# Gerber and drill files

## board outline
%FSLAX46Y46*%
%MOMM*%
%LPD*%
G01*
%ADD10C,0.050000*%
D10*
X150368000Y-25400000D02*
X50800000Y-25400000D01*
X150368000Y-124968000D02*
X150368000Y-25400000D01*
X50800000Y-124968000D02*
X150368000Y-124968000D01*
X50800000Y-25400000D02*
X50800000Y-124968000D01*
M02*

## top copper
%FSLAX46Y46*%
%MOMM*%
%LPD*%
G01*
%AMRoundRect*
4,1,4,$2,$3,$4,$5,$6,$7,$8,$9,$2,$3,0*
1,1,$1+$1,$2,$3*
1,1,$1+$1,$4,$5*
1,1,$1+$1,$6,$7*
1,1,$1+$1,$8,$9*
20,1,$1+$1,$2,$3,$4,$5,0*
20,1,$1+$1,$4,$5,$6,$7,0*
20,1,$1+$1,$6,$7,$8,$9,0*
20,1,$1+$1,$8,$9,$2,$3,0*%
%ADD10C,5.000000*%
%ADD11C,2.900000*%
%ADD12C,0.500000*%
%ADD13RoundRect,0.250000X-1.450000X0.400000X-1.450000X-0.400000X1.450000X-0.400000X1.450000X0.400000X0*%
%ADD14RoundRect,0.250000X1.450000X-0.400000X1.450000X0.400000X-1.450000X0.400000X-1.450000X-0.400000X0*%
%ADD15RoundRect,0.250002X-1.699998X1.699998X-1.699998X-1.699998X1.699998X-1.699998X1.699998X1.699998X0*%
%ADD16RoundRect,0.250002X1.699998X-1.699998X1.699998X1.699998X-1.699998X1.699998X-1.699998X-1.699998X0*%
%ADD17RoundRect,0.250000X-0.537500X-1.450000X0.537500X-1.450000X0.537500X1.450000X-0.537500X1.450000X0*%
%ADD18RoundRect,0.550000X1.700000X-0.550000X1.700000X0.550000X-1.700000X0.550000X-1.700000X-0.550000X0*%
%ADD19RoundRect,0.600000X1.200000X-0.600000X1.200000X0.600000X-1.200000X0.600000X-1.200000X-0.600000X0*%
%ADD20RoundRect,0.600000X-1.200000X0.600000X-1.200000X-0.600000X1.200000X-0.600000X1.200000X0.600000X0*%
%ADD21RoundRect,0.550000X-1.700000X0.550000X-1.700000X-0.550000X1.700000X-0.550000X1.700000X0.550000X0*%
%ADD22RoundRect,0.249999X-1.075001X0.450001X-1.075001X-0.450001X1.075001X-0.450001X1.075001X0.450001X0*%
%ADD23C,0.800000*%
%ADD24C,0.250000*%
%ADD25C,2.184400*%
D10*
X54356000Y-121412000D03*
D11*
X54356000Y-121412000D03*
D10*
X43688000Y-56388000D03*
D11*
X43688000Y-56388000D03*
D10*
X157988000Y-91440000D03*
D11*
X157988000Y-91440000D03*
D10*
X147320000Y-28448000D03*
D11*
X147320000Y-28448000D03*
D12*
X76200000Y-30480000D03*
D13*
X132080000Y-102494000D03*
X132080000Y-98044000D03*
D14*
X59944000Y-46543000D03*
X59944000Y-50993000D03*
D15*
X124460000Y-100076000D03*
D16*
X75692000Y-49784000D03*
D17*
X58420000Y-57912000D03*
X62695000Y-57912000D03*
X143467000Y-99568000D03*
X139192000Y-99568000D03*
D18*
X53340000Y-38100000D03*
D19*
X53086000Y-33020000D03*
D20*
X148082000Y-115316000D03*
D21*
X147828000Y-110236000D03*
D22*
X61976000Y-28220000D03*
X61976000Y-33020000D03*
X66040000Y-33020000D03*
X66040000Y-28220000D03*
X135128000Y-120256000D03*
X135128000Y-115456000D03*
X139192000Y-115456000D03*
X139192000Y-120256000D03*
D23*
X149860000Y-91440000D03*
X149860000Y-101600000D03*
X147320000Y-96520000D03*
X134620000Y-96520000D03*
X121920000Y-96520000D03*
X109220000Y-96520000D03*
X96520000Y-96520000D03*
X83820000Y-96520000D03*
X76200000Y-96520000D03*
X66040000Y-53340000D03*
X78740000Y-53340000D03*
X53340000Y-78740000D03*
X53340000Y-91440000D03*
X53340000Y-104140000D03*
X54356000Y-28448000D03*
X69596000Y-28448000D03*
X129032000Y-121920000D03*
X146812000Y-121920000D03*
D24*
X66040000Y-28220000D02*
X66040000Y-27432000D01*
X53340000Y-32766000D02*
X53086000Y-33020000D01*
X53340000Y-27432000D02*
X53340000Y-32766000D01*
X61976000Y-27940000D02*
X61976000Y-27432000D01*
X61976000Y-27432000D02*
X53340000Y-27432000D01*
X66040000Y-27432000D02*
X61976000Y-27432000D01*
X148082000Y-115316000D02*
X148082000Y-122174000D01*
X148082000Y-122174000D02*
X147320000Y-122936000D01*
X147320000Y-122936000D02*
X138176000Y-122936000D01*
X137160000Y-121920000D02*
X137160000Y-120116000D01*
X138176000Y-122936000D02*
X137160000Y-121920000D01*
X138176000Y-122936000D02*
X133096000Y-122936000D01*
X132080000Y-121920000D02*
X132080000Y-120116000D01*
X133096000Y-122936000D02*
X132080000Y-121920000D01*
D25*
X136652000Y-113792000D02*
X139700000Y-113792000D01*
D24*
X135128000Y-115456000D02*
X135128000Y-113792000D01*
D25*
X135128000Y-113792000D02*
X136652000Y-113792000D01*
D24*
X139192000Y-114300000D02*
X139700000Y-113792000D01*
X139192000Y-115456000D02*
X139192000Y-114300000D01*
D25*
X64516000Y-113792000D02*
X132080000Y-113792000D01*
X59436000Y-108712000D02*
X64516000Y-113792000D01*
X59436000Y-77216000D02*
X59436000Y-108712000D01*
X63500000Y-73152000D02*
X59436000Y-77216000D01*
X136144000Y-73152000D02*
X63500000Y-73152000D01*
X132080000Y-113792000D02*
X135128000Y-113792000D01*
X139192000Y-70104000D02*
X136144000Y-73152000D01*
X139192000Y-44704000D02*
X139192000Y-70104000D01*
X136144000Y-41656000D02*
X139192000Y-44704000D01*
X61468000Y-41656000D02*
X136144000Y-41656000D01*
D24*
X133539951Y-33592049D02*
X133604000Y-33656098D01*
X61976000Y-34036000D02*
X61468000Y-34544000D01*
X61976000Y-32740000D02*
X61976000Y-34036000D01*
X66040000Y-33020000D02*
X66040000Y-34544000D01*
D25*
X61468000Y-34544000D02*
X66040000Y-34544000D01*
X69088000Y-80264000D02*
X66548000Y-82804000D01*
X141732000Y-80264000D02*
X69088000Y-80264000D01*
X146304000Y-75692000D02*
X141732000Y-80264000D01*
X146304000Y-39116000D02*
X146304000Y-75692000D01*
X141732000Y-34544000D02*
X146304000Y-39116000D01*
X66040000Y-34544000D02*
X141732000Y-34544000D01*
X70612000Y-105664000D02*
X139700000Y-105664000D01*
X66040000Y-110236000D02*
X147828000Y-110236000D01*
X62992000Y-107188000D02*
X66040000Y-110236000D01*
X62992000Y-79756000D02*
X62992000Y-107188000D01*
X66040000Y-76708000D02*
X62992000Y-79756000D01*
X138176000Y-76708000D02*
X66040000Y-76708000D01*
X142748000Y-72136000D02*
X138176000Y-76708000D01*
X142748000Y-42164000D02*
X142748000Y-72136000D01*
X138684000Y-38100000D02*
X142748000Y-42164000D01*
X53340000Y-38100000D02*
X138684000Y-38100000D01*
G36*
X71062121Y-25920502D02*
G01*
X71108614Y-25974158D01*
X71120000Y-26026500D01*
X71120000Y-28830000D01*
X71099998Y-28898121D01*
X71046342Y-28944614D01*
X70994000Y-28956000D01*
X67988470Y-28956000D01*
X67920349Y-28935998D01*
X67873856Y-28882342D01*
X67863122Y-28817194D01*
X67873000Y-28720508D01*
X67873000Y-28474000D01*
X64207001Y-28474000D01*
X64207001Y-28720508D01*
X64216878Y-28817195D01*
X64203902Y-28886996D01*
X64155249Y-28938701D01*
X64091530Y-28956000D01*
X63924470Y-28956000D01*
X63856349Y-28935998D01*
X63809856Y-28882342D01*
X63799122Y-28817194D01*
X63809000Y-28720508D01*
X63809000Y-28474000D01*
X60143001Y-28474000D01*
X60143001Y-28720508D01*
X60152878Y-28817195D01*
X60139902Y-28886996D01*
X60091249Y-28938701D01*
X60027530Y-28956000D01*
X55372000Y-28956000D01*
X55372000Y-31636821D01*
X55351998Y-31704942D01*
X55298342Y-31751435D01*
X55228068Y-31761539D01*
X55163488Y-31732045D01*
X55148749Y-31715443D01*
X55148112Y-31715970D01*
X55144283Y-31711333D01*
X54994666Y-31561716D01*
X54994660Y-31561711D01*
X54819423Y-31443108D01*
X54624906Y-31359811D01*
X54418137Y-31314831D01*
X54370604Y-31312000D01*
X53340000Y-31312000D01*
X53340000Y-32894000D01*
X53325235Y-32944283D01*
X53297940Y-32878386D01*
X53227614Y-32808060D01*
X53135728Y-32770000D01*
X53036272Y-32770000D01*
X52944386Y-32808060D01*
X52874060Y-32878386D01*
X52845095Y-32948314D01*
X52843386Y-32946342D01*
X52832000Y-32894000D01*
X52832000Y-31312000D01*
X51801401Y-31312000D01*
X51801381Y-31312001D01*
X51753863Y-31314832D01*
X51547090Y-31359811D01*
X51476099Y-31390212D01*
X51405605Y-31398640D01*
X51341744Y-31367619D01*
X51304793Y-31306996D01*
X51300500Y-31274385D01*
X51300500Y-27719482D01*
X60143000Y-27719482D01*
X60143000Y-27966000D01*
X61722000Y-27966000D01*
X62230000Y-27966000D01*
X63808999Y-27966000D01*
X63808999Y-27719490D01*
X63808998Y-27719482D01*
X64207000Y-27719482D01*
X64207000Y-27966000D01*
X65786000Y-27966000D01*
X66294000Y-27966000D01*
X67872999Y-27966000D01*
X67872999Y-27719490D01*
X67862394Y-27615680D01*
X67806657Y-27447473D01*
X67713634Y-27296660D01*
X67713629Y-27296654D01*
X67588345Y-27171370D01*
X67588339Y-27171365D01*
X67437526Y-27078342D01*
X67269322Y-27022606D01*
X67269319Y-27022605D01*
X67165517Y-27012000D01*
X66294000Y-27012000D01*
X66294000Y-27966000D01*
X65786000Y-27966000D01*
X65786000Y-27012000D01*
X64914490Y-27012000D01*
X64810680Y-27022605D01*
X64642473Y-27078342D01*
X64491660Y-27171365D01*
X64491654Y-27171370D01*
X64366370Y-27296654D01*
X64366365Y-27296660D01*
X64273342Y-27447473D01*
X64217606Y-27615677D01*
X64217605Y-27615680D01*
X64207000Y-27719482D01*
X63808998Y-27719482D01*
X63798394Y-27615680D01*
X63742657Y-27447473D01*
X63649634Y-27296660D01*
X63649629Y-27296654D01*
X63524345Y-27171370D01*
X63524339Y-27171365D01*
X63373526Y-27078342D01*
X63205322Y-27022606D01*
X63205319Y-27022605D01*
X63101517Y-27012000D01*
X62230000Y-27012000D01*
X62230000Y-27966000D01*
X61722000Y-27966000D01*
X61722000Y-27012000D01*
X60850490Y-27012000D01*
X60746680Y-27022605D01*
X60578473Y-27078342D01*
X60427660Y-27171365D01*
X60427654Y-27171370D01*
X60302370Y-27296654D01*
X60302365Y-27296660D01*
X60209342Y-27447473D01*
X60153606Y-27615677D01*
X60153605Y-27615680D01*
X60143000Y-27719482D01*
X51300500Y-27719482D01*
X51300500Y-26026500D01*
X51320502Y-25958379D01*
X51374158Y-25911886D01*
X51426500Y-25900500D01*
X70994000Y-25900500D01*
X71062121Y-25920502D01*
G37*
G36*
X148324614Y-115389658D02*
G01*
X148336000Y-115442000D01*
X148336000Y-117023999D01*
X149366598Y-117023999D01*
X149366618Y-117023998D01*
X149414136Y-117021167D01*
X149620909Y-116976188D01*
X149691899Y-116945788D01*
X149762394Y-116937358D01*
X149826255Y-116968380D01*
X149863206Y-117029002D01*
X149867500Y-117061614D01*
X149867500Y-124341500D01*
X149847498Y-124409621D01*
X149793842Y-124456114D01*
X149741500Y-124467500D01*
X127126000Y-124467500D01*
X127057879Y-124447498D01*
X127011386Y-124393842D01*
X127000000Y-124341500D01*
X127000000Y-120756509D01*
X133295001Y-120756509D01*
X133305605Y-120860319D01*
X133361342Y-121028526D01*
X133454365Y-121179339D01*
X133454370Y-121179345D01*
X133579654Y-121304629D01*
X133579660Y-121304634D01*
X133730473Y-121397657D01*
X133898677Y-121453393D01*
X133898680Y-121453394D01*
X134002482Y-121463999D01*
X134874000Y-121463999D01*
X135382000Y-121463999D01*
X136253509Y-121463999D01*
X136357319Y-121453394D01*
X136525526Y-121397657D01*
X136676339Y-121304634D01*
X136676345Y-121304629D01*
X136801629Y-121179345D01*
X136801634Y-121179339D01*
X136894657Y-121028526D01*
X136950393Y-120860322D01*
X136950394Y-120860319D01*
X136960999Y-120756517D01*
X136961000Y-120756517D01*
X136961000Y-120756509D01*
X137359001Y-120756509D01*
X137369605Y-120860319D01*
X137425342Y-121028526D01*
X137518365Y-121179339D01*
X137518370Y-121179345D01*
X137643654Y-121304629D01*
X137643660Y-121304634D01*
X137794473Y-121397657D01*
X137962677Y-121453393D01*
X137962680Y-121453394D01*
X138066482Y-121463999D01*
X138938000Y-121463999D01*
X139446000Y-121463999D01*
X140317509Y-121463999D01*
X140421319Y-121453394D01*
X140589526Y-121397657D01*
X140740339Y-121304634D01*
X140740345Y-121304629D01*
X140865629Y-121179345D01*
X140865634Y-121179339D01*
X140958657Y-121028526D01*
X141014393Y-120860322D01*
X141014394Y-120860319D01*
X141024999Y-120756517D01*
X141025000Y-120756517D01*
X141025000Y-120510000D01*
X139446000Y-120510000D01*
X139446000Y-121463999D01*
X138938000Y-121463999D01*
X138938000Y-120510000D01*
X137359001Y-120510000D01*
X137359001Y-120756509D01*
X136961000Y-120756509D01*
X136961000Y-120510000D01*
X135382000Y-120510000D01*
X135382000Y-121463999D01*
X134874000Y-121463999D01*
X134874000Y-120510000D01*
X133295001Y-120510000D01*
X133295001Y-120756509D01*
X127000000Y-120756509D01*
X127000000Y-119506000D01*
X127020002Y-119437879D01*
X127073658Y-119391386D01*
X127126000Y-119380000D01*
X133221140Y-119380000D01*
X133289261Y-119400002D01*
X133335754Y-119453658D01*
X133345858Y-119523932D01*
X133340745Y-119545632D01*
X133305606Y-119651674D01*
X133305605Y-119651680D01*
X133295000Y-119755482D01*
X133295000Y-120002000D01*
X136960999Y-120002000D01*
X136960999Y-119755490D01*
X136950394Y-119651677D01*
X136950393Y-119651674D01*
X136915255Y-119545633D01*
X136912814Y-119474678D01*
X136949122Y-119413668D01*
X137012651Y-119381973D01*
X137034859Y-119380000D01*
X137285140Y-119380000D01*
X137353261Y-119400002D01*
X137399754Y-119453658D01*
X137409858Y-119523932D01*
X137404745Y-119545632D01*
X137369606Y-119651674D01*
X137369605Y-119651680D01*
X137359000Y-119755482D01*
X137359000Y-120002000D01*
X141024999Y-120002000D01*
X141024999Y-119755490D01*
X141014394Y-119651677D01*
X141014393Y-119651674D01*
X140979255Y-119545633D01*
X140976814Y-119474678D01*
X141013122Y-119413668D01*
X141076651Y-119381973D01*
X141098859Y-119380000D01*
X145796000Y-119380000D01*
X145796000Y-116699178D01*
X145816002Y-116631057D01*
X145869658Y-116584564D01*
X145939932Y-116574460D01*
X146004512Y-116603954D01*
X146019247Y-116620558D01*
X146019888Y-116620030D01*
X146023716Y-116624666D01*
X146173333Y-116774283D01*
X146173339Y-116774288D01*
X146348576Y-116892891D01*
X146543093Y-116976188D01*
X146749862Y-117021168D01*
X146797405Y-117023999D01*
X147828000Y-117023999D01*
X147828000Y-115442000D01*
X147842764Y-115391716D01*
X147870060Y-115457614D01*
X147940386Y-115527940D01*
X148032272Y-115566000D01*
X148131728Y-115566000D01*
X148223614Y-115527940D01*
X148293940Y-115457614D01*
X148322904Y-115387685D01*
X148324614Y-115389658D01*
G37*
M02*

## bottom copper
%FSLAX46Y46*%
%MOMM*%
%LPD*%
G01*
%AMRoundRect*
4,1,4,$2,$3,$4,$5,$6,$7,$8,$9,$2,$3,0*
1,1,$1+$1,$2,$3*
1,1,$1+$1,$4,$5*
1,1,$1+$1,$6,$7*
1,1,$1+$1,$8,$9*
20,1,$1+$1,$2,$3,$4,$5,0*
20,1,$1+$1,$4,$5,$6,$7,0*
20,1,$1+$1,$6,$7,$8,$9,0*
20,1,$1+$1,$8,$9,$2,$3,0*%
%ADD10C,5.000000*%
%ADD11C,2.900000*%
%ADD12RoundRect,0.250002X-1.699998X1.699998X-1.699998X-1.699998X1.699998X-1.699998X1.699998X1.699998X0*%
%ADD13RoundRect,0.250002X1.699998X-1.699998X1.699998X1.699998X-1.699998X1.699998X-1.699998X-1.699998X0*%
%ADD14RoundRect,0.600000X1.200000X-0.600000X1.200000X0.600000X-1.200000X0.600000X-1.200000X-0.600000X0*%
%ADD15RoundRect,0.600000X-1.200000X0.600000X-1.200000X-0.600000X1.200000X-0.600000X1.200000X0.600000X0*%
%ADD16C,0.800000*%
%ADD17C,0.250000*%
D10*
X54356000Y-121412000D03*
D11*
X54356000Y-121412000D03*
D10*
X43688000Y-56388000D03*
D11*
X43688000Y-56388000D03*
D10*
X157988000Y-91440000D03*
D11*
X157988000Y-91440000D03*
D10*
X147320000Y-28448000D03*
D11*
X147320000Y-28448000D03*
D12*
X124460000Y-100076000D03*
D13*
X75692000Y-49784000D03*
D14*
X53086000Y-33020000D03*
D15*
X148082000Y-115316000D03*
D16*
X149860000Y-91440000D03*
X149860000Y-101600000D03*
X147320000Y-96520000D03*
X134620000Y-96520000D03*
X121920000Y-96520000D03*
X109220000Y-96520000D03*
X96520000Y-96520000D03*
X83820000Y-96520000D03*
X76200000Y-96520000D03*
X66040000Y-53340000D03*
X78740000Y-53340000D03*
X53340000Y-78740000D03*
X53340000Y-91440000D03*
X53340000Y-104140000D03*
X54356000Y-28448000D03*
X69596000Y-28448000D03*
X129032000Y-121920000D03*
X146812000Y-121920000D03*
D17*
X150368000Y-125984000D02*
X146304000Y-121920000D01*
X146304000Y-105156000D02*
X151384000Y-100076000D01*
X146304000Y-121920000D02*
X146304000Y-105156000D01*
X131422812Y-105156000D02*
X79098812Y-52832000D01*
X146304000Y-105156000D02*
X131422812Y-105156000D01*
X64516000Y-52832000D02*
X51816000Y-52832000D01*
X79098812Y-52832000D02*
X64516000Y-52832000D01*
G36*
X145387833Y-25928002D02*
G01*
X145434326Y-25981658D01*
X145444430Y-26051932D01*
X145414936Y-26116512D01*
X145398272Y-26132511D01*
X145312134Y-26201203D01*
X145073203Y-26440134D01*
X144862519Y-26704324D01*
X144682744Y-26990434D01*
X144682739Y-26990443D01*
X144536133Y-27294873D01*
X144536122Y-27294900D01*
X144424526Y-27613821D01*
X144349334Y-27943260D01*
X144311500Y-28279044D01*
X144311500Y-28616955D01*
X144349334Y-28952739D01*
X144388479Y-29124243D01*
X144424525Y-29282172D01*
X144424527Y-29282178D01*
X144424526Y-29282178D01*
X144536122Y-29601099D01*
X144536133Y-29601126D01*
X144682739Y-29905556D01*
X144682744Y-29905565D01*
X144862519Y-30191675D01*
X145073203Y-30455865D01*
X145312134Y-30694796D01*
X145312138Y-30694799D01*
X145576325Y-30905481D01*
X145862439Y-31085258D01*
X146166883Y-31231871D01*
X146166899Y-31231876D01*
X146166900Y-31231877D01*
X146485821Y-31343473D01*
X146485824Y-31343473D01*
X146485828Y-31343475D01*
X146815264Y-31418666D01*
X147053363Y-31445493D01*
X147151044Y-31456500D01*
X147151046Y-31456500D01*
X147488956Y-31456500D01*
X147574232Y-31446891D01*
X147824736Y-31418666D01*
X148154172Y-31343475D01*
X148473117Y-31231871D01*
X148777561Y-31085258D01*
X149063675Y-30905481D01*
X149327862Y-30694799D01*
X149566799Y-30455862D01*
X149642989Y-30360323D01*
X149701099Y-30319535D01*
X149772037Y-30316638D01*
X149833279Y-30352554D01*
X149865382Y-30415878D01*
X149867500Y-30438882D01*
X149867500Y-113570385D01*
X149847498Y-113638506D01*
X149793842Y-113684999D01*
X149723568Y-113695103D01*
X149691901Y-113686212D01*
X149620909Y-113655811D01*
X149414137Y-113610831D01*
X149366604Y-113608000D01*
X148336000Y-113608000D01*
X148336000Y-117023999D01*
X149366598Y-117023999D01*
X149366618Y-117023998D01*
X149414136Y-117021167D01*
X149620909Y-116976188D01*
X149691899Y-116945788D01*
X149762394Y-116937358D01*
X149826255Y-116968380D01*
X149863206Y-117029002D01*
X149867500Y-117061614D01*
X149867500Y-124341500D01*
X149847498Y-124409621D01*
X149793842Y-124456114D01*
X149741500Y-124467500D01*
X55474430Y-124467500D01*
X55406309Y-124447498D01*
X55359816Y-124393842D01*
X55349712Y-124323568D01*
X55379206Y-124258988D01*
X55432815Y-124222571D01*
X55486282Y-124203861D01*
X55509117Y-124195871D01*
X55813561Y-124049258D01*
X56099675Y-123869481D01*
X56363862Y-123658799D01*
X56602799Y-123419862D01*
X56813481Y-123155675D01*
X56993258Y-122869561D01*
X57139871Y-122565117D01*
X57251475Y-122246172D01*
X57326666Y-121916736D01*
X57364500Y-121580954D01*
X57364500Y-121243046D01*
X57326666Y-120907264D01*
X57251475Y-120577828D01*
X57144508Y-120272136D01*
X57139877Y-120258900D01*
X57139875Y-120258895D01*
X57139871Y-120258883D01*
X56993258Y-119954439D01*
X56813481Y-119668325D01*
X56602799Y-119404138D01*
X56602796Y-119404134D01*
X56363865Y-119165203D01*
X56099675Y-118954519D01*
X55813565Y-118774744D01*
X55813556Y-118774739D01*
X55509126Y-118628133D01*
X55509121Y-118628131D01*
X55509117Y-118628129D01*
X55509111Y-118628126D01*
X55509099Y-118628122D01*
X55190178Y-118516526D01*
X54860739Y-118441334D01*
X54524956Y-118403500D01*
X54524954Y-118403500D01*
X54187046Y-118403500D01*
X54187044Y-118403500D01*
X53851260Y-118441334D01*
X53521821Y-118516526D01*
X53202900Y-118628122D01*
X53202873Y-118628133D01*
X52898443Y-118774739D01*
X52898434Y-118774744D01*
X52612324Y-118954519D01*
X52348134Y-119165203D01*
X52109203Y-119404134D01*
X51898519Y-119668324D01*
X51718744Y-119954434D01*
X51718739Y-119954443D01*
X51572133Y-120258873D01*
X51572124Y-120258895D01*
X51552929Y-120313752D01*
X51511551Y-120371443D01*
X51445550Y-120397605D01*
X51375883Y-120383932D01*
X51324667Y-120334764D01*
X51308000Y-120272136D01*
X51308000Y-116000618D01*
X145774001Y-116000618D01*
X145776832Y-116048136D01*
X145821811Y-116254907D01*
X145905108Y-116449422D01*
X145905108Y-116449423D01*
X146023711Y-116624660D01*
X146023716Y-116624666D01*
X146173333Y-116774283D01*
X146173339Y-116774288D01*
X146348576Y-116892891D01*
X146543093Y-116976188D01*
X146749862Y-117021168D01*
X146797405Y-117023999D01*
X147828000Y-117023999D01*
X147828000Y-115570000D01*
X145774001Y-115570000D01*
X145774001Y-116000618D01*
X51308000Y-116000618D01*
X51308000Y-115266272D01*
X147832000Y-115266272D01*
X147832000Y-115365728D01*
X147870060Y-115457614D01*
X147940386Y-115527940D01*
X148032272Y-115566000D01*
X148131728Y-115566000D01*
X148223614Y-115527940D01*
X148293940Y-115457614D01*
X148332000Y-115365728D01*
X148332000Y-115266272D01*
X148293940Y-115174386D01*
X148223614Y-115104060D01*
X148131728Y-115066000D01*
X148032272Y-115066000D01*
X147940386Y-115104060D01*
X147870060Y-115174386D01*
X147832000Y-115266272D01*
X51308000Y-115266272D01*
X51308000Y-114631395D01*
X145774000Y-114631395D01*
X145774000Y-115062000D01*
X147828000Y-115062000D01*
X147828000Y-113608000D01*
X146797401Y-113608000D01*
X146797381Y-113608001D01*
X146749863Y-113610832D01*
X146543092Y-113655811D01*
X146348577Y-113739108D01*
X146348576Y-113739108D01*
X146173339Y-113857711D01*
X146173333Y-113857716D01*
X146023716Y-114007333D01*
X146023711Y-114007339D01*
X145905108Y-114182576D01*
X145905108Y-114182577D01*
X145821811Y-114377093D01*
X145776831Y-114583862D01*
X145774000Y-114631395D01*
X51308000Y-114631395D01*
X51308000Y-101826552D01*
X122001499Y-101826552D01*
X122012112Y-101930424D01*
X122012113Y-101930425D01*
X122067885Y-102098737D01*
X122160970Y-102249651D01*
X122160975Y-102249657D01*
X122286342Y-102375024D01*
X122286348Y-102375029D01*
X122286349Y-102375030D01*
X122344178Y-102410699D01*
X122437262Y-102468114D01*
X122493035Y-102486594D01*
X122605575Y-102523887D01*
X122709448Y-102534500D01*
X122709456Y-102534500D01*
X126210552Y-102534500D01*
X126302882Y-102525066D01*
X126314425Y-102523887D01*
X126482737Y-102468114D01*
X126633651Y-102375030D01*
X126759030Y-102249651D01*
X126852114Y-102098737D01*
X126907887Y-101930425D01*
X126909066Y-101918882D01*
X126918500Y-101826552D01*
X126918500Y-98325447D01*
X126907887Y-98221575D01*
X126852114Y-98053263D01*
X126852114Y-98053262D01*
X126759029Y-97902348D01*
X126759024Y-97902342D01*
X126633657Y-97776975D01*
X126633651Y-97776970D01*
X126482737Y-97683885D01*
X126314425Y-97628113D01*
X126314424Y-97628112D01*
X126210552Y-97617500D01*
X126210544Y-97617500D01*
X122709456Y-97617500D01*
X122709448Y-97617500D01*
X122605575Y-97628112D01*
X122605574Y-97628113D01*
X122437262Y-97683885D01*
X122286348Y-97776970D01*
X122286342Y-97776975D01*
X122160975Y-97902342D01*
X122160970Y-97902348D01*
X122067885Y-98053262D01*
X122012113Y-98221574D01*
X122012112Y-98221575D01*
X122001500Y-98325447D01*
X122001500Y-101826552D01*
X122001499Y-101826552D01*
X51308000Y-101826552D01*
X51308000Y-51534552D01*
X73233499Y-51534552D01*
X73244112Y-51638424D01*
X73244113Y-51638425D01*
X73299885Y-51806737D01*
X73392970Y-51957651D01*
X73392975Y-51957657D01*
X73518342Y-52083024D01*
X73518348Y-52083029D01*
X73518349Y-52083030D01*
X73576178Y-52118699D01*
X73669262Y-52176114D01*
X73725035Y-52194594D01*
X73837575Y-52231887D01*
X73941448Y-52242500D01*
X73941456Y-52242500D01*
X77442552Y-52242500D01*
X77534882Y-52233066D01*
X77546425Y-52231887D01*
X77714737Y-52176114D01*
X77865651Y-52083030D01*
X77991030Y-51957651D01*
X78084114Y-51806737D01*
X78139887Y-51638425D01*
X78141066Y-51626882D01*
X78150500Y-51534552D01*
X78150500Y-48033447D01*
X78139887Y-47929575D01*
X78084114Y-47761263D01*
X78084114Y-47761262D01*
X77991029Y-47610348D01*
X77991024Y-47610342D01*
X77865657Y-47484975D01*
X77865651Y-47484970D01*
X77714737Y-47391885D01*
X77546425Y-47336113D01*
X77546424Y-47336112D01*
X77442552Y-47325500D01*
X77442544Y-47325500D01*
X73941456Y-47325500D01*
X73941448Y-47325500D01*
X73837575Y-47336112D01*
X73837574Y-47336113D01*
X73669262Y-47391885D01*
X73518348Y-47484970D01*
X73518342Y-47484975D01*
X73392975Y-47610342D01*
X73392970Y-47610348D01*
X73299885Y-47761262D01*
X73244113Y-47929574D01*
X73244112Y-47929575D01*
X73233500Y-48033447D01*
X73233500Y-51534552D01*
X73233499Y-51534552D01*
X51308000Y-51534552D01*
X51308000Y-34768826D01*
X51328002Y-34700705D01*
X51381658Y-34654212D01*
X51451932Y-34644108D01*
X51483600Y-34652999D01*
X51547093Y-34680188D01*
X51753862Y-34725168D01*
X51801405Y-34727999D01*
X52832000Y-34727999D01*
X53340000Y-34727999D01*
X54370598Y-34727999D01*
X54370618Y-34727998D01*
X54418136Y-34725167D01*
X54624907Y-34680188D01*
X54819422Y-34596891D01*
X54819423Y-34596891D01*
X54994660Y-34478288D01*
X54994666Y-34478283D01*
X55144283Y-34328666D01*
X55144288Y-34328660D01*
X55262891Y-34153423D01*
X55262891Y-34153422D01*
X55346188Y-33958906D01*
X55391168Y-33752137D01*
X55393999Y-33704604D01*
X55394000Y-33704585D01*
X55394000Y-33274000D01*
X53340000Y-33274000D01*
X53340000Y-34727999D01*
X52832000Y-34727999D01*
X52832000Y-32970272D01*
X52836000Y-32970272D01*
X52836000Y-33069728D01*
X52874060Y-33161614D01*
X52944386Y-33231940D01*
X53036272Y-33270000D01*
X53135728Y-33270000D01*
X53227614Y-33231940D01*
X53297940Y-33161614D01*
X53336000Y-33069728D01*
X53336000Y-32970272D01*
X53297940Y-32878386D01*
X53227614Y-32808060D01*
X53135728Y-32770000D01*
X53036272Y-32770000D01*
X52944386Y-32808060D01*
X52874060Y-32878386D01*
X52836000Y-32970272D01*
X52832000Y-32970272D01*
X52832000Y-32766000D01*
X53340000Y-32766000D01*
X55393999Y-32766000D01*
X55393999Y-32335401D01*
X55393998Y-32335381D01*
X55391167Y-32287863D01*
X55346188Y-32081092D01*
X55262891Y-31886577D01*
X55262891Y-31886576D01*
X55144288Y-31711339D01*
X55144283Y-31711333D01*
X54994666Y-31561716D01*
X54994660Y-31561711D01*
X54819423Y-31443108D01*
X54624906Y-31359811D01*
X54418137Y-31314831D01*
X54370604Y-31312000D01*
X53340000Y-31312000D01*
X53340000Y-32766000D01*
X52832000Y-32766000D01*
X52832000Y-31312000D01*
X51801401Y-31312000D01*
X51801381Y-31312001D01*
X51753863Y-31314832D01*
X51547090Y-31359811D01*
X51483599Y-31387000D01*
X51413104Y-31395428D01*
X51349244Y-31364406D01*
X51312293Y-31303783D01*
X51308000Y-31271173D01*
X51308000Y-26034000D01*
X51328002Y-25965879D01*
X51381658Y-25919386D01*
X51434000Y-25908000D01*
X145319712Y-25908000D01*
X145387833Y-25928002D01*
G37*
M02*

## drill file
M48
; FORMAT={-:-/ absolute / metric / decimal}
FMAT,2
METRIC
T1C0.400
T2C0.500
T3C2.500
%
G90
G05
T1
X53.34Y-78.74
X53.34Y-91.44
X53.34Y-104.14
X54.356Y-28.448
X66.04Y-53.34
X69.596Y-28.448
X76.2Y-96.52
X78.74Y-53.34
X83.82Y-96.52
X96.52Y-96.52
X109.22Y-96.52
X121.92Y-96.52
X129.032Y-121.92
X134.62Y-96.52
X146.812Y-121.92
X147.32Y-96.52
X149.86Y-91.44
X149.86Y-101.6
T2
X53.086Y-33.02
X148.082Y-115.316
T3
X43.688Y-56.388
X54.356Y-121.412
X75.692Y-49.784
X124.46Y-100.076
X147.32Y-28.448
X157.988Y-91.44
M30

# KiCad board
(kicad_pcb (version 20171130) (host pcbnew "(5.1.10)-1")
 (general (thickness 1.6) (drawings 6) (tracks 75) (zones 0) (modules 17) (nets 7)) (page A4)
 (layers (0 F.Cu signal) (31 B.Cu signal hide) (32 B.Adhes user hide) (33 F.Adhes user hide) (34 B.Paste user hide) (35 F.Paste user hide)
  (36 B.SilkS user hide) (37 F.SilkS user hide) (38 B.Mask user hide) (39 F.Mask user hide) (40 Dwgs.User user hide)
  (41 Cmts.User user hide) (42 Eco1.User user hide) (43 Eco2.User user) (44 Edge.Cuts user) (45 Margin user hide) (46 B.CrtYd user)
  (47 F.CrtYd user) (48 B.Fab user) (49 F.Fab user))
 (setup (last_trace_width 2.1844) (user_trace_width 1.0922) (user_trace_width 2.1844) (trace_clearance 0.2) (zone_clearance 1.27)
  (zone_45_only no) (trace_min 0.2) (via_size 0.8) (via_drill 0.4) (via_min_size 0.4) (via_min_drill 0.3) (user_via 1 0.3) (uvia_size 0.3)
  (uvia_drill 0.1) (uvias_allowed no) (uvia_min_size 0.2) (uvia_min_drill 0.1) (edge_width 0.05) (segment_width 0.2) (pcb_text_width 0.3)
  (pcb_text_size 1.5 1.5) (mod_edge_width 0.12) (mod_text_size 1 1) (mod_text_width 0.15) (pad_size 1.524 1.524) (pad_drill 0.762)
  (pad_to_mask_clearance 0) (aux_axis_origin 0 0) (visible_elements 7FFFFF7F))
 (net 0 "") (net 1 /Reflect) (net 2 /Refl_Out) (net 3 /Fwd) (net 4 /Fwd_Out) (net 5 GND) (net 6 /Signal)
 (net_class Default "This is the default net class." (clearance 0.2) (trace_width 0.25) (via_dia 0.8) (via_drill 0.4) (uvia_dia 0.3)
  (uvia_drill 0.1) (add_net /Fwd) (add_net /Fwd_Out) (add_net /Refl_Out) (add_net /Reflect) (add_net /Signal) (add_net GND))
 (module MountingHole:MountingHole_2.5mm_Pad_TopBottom (layer F.Cu) (at 54.356 121.412)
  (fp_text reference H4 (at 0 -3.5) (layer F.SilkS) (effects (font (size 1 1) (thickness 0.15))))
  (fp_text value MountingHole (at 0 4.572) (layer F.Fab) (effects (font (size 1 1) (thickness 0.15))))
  (pad 1 connect circle (at 0 0) (size 5 5) (layers B.Cu B.Mask))
  (pad 1 connect circle (at 0 0) (size 5 5) (layers F.Cu F.Mask))
  (pad 1 thru_hole circle (at 0 0) (size 2.9 2.9) (drill 2.5) (layers *.Cu *.Mask)))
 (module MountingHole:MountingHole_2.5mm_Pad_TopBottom (layer F.Cu) (at 43.688 56.388)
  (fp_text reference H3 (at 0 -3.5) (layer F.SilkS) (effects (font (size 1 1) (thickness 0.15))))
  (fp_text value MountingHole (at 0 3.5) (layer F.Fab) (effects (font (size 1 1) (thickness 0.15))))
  (pad 1 connect circle (at 0 0) (size 5 5) (layers B.Cu B.Mask))
  (pad 1 connect circle (at 0 0) (size 5 5) (layers F.Cu F.Mask))
  (pad 1 thru_hole circle (at 0 0) (size 2.9 2.9) (drill 2.5) (layers *.Cu *.Mask)))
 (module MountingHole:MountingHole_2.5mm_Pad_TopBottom (layer F.Cu) (at 157.988 91.44)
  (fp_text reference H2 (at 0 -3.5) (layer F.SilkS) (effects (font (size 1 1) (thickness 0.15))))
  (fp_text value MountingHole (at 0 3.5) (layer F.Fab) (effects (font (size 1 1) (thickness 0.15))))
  (pad 1 connect circle (at 0 0) (size 5 5) (layers B.Cu B.Mask))
  (pad 1 connect circle (at 0 0) (size 5 5) (layers F.Cu F.Mask))
  (pad 1 thru_hole circle (at 0 0) (size 2.9 2.9) (drill 2.5) (layers *.Cu *.Mask)))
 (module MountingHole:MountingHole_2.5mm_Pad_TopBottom (layer F.Cu) (at 147.32 28.448)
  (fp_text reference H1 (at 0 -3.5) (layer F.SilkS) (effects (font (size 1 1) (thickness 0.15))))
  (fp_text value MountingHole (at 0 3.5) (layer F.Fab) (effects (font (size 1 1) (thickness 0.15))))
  (pad 1 connect circle (at 0 0) (size 5 5) (layers B.Cu B.Mask))
  (pad 1 connect circle (at 0 0) (size 5 5) (layers F.Cu F.Mask))
  (pad 1 thru_hole circle (at 0 0) (size 2.9 2.9) (drill 2.5) (layers *.Cu *.Mask)))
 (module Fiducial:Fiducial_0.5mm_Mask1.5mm (layer F.Cu) (at 76.2 30.48)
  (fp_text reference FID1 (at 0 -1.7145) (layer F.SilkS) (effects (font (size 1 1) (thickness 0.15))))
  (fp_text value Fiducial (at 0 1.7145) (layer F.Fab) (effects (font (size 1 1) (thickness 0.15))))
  (pad "" smd circle (at 0 0) (size 0.5 0.5) (layers F.Cu F.Mask) (solder_mask_margin 0.5) (clearance 0.5)))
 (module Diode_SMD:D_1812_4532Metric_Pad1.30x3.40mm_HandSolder (layer F.Cu) (at 132.08 100.269 270)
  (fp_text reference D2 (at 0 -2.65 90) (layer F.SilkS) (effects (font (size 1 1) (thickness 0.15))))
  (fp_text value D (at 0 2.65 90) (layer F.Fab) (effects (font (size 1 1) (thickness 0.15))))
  (pad 2 smd roundrect (at 2.225 0 270) (size 1.3 3.4) (layers F.Cu F.Paste F.Mask) (roundrect_rratio 0.192308) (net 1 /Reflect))
  (pad 1 smd roundrect (at -2.225 0 270) (size 1.3 3.4) (layers F.Cu F.Paste F.Mask) (roundrect_rratio 0.192308) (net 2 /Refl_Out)))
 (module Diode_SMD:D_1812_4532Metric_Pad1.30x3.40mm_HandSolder (layer F.Cu) (at 59.944 48.768 90)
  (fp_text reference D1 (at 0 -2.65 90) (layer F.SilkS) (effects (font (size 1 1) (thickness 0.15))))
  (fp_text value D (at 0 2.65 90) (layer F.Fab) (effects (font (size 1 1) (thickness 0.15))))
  (pad 2 smd roundrect (at 2.225 0 90) (size 1.3 3.4) (layers F.Cu F.Paste F.Mask) (roundrect_rratio 0.192308) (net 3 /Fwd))
  (pad 1 smd roundrect (at -2.225 0 90) (size 1.3 3.4) (layers F.Cu F.Paste F.Mask) (roundrect_rratio 0.192308) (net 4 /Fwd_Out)))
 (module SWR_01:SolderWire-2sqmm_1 (layer F.Cu) (at 124.46 100.076 270)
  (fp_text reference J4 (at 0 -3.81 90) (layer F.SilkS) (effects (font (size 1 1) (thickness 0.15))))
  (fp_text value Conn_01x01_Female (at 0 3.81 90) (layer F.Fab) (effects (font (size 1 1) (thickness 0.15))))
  (pad 1 thru_hole roundrect (at 0 0 270) (size 3.9 3.9) (drill 2.5) (layers *.Cu *.Mask) (roundrect_rratio 0.06410299999999999)
   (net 2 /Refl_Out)))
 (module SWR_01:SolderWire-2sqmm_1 (layer F.Cu) (at 75.692 49.784 90)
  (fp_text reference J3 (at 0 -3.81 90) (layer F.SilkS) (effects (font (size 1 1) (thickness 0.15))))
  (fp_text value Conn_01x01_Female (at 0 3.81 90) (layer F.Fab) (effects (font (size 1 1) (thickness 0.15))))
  (pad 1 thru_hole roundrect (at 0 0 90) (size 3.9 3.9) (drill 2.5) (layers *.Cu *.Mask) (roundrect_rratio 0.06410299999999999)
   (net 4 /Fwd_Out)))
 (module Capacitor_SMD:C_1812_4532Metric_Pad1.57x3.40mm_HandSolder (layer F.Cu) (at 60.5575 57.912)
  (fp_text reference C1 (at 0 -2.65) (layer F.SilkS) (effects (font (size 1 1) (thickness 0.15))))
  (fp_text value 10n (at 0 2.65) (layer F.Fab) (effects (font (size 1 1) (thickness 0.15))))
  (pad 1 smd roundrect (at -2.1375 0) (size 1.575 3.4) (layers F.Cu F.Paste F.Mask) (roundrect_rratio 0.15873) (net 4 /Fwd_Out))
  (pad 2 smd roundrect (at 2.1375 0) (size 1.575 3.4) (layers F.Cu F.Paste F.Mask) (roundrect_rratio 0.15873) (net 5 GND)))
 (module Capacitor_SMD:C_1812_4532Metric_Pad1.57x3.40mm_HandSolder (layer F.Cu) (at 141.3295 99.568)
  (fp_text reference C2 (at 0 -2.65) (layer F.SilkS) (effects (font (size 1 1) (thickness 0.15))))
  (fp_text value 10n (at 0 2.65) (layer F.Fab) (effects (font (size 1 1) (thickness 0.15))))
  (pad 2 smd roundrect (at 2.1375 0) (size 1.575 3.4) (layers F.Cu F.Paste F.Mask) (roundrect_rratio 0.15873) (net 2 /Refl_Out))
  (pad 1 smd roundrect (at -2.1375 0) (size 1.575 3.4) (layers F.Cu F.Paste F.Mask) (roundrect_rratio 0.15873) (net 5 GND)))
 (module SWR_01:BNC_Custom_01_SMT (layer F.Cu) (at 54.356 38.1 90)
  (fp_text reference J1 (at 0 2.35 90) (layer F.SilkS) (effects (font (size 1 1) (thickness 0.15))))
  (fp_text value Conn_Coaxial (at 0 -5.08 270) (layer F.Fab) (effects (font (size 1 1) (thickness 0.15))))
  (pad 1 connect roundrect (at 0 -1.016 90) (size 2.2 4.5) (layers F.Cu F.Mask) (roundrect_rratio 0.25) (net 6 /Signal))
  (pad 2 thru_hole roundrect (at 5.08 -1.27 90) (size 2.4 3.6) (drill 0.5) (layers *.Cu *.Mask) (roundrect_rratio 0.25) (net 5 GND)))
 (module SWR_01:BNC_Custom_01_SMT (layer F.Cu) (at 146.812 110.236 270)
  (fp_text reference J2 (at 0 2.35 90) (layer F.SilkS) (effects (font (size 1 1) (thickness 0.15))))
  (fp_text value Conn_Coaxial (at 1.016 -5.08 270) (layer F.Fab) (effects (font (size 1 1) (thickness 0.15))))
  (pad 2 thru_hole roundrect (at 5.08 -1.27 270) (size 2.4 3.6) (drill 0.5) (layers *.Cu *.Mask) (roundrect_rratio 0.25) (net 5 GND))
  (pad 1 connect roundrect (at 0 -1.016 270) (size 2.2 4.5) (layers F.Cu F.Mask) (roundrect_rratio 0.25) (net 6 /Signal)))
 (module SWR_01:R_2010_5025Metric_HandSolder (layer F.Cu) (at 61.976 30.62 270)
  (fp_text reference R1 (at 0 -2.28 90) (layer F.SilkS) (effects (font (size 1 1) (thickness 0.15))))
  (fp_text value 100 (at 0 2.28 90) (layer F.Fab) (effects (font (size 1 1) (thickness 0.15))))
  (pad 1 smd roundrect (at -2.4 0 270) (size 1.4 2.65) (layers F.Cu F.Paste F.Mask) (roundrect_rratio 0.178571) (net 5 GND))
  (pad 2 smd roundrect (at 2.4 0 270) (size 1.4 2.65) (layers F.Cu F.Paste F.Mask) (roundrect_rratio 0.178571) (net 1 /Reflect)))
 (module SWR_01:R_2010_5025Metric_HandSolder (layer F.Cu) (at 66.04 30.62 270)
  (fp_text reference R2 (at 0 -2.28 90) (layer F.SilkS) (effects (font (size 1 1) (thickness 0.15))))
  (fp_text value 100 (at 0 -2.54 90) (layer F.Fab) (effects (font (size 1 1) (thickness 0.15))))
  (pad 2 smd roundrect (at 2.4 0 270) (size 1.4 2.65) (layers F.Cu F.Paste F.Mask) (roundrect_rratio 0.178571) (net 1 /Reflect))
  (pad 1 smd roundrect (at -2.4 0 270) (size 1.4 2.65) (layers F.Cu F.Paste F.Mask) (roundrect_rratio 0.178571) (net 5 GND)))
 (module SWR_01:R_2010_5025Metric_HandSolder (layer F.Cu) (at 135.128 117.856 270)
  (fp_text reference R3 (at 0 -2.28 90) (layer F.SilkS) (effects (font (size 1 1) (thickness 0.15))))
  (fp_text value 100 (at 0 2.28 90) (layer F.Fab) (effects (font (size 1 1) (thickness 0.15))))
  (pad 2 smd roundrect (at 2.4 0 270) (size 1.4 2.65) (layers F.Cu F.Paste F.Mask) (roundrect_rratio 0.178571) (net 5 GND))
  (pad 1 smd roundrect (at -2.4 0 270) (size 1.4 2.65) (layers F.Cu F.Paste F.Mask) (roundrect_rratio 0.178571) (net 3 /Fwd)))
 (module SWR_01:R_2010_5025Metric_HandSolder (layer F.Cu) (at 139.192 117.856 270)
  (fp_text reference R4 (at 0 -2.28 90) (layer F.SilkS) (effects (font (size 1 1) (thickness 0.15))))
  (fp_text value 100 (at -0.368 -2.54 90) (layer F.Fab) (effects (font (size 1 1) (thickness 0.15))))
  (pad 1 smd roundrect (at -2.4 0 270) (size 1.4 2.65) (layers F.Cu F.Paste F.Mask) (roundrect_rratio 0.178571) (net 3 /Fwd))
  (pad 2 smd roundrect (at 2.4 0 270) (size 1.4 2.65) (layers F.Cu F.Paste F.Mask) (roundrect_rratio 0.178571) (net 5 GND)))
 (gr_line (start 150.368 25.4) (end 50.8 25.4) (layer Edge.Cuts) (width 0.05))
 (gr_line (start 150.368 124.968) (end 150.368 25.4) (layer Edge.Cuts) (width 0.05))
 (gr_line (start 50.8 124.968) (end 150.368 124.968) (layer Edge.Cuts) (width 0.05))
 (gr_line (start 50.8 25.4) (end 50.8 124.968) (layer Edge.Cuts) (width 0.05))
 (segment (start 150.368 125.984) (end 146.304 121.92) (width 0.25) (layer B.Cu) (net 5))
 (segment (start 146.304 105.156) (end 151.384 100.076) (width 0.25) (layer B.Cu) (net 5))
 (segment (start 146.304 121.92) (end 146.304 105.156) (width 0.25) (layer B.Cu) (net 5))
 (segment (start 131.422812 105.156) (end 79.098812 52.832) (width 0.25) (layer B.Cu) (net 5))
 (segment (start 146.304 105.156) (end 131.422812 105.156) (width 0.25) (layer B.Cu) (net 5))
 (segment (start 64.516 52.832) (end 51.816 52.832) (width 0.25) (layer B.Cu) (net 5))
 (segment (start 79.098812 52.832) (end 64.516 52.832) (width 0.25) (layer B.Cu) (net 5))
 (via (at 149.86 91.44) (size 0.8) (drill 0.4) (layers F.Cu B.Cu) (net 5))
 (via (at 149.86 101.6) (size 0.8) (drill 0.4) (layers F.Cu B.Cu) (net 5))
 (via (at 147.32 96.52) (size 0.8) (drill 0.4) (layers F.Cu B.Cu) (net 5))
 (via (at 134.62 96.52) (size 0.8) (drill 0.4) (layers F.Cu B.Cu) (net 5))
 (via (at 121.92 96.52) (size 0.8) (drill 0.4) (layers F.Cu B.Cu) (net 5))
 (via (at 109.22 96.52) (size 0.8) (drill 0.4) (layers F.Cu B.Cu) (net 5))
 (via (at 96.52 96.52) (size 0.8) (drill 0.4) (layers F.Cu B.Cu) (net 5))
 (via (at 83.82 96.52) (size 0.8) (drill 0.4) (layers F.Cu B.Cu) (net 5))
 (via (at 76.2 96.52) (size 0.8) (drill 0.4) (layers F.Cu B.Cu) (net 5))
 (via (at 66.04 53.34) (size 0.8) (drill 0.4) (layers F.Cu B.Cu) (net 5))
 (via (at 78.74 53.34) (size 0.8) (drill 0.4) (layers F.Cu B.Cu) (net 5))
 (via (at 53.34 78.74) (size 0.8) (drill 0.4) (layers F.Cu B.Cu) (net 5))
 (via (at 53.34 91.44) (size 0.8) (drill 0.4) (layers F.Cu B.Cu) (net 5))
 (via (at 53.34 104.14) (size 0.8) (drill 0.4) (layers F.Cu B.Cu) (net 5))
 (segment (start 66.04 28.22) (end 66.04 27.432) (width 0.25) (layer F.Cu) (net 5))
 (segment (start 53.34 32.766) (end 53.086 33.02) (width 0.25) (layer F.Cu) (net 5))
 (segment (start 53.34 27.432) (end 53.34 32.766) (width 0.25) (layer F.Cu) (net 5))
 (segment (start 61.976 27.94) (end 61.976 27.432) (width 0.25) (layer F.Cu) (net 5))
 (segment (start 61.976 27.432) (end 53.34 27.432) (width 0.25) (layer F.Cu) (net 5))
 (segment (start 66.04 27.432) (end 61.976 27.432) (width 0.25) (layer F.Cu) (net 5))
 (via (at 54.356 28.448) (size 0.8) (drill 0.4) (layers F.Cu B.Cu) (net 5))
 (via (at 69.596 28.448) (size 0.8) (drill 0.4) (layers F.Cu B.Cu) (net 5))
 (segment (start 148.082 115.316) (end 148.082 122.174) (width 0.25) (layer F.Cu) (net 5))
 (segment (start 148.082 122.174) (end 147.32 122.936) (width 0.25) (layer F.Cu) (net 5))
 (segment (start 147.32 122.936) (end 138.176 122.936) (width 0.25) (layer F.Cu) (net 5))
 (segment (start 137.16 121.92) (end 137.16 120.116) (width 0.25) (layer F.Cu) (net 5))
 (segment (start 138.176 122.936) (end 137.16 121.92) (width 0.25) (layer F.Cu) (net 5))
 (segment (start 138.176 122.936) (end 133.096 122.936) (width 0.25) (layer F.Cu) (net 5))
 (segment (start 132.08 121.92) (end 132.08 120.116) (width 0.25) (layer F.Cu) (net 5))
 (segment (start 133.096 122.936) (end 132.08 121.92) (width 0.25) (layer F.Cu) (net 5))
 (via (at 129.032 121.92) (size 0.8) (drill 0.4) (layers F.Cu B.Cu) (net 5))
 (via (at 146.812 121.92) (size 0.8) (drill 0.4) (layers F.Cu B.Cu) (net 5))
 (segment (start 136.652 113.792) (end 139.7 113.792) (width 2.1844) (layer F.Cu) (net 3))
 (segment (start 135.128 115.456) (end 135.128 113.792) (width 0.25) (layer F.Cu) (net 3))
 (segment (start 135.128 113.792) (end 136.652 113.792) (width 2.1844) (layer F.Cu) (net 3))
 (segment (start 139.192 114.3) (end 139.7 113.792) (width 0.25) (layer F.Cu) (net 3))
 (segment (start 139.192 115.456) (end 139.192 114.3) (width 0.25) (layer F.Cu) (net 3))
 (segment (start 64.516 113.792) (end 132.08 113.792) (width 2.1844) (layer F.Cu) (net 3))
 (segment (start 59.436 108.712) (end 64.516 113.792) (width 2.1844) (layer F.Cu) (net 3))
 (segment (start 59.436 77.216) (end 59.436 108.712) (width 2.1844) (layer F.Cu) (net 3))
 (segment (start 63.5 73.152) (end 59.436 77.216) (width 2.1844) (layer F.Cu) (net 3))
 (segment (start 136.144 73.152) (end 63.5 73.152) (width 2.1844) (layer F.Cu) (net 3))
 (segment (start 132.08 113.792) (end 135.128 113.792) (width 2.1844) (layer F.Cu) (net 3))
 (segment (start 139.192 70.104) (end 136.144 73.152) (width 2.1844) (layer F.Cu) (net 3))
 (segment (start 139.192 44.704) (end 139.192 70.104) (width 2.1844) (layer F.Cu) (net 3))
 (segment (start 136.144 41.656) (end 139.192 44.704) (width 2.1844) (layer F.Cu) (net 3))
 (segment (start 61.468 41.656) (end 136.144 41.656) (width 2.1844) (layer F.Cu) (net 3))
 (segment (start 133.539951 33.592049) (end 133.604 33.656098) (width 0.25) (layer F.Cu) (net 1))
 (segment (start 61.976 34.036) (end 61.468 34.544) (width 0.25) (layer F.Cu) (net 1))
 (segment (start 61.976 32.74) (end 61.976 34.036) (width 0.25) (layer F.Cu) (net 1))
 (segment (start 66.04 33.02) (end 66.04 34.544) (width 0.25) (layer F.Cu) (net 1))
 (segment (start 61.468 34.544) (end 66.04 34.544) (width 2.1844) (layer F.Cu) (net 1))
 (segment (start 69.088 80.264) (end 66.548 82.804) (width 2.1844) (layer F.Cu) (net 1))
 (segment (start 141.732 80.264) (end 69.088 80.264) (width 2.1844) (layer F.Cu) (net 1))
 (segment (start 146.304 75.692) (end 141.732 80.264) (width 2.1844) (layer F.Cu) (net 1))
 (segment (start 146.304 39.116) (end 146.304 75.692) (width 2.1844) (layer F.Cu) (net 1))
 (segment (start 141.732 34.544) (end 146.304 39.116) (width 2.1844) (layer F.Cu) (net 1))
 (segment (start 66.04 34.544) (end 141.732 34.544) (width 2.1844) (layer F.Cu) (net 1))
 (segment (start 70.612 105.664) (end 139.7 105.664) (width 2.1844) (layer F.Cu) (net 1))
 (segment (start 66.04 110.236) (end 147.828 110.236) (width 2.1844) (layer F.Cu) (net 6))
 (segment (start 62.992 107.188) (end 66.04 110.236) (width 2.1844) (layer F.Cu) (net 6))
 (segment (start 62.992 79.756) (end 62.992 107.188) (width 2.1844) (layer F.Cu) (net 6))
 (segment (start 66.04 76.708) (end 62.992 79.756) (width 2.1844) (layer F.Cu) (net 6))
 (segment (start 138.176 76.708) (end 66.04 76.708) (width 2.1844) (layer F.Cu) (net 6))
 (segment (start 142.748 72.136) (end 138.176 76.708) (width 2.1844) (layer F.Cu) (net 6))
 (segment (start 142.748 42.164) (end 142.748 72.136) (width 2.1844) (layer F.Cu) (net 6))
 (segment (start 138.684 38.1) (end 142.748 42.164) (width 2.1844) (layer F.Cu) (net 6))
 (segment (start 53.34 38.1) (end 138.684 38.1) (width 2.1844) (layer F.Cu) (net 6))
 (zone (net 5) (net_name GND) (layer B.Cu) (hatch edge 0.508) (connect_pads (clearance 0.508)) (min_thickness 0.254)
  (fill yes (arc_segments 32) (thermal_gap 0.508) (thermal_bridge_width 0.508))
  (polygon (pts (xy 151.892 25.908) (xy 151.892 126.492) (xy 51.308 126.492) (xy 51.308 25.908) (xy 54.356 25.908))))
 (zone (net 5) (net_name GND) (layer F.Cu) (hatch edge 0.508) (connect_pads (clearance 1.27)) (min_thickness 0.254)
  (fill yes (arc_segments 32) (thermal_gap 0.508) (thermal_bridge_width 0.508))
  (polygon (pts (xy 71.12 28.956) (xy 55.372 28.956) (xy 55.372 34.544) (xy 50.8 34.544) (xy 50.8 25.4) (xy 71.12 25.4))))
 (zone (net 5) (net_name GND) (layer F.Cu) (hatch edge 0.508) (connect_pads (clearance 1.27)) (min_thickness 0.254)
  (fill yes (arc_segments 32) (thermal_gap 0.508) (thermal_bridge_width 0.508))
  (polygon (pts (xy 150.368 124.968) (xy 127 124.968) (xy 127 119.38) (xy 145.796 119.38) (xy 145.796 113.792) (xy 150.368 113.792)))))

